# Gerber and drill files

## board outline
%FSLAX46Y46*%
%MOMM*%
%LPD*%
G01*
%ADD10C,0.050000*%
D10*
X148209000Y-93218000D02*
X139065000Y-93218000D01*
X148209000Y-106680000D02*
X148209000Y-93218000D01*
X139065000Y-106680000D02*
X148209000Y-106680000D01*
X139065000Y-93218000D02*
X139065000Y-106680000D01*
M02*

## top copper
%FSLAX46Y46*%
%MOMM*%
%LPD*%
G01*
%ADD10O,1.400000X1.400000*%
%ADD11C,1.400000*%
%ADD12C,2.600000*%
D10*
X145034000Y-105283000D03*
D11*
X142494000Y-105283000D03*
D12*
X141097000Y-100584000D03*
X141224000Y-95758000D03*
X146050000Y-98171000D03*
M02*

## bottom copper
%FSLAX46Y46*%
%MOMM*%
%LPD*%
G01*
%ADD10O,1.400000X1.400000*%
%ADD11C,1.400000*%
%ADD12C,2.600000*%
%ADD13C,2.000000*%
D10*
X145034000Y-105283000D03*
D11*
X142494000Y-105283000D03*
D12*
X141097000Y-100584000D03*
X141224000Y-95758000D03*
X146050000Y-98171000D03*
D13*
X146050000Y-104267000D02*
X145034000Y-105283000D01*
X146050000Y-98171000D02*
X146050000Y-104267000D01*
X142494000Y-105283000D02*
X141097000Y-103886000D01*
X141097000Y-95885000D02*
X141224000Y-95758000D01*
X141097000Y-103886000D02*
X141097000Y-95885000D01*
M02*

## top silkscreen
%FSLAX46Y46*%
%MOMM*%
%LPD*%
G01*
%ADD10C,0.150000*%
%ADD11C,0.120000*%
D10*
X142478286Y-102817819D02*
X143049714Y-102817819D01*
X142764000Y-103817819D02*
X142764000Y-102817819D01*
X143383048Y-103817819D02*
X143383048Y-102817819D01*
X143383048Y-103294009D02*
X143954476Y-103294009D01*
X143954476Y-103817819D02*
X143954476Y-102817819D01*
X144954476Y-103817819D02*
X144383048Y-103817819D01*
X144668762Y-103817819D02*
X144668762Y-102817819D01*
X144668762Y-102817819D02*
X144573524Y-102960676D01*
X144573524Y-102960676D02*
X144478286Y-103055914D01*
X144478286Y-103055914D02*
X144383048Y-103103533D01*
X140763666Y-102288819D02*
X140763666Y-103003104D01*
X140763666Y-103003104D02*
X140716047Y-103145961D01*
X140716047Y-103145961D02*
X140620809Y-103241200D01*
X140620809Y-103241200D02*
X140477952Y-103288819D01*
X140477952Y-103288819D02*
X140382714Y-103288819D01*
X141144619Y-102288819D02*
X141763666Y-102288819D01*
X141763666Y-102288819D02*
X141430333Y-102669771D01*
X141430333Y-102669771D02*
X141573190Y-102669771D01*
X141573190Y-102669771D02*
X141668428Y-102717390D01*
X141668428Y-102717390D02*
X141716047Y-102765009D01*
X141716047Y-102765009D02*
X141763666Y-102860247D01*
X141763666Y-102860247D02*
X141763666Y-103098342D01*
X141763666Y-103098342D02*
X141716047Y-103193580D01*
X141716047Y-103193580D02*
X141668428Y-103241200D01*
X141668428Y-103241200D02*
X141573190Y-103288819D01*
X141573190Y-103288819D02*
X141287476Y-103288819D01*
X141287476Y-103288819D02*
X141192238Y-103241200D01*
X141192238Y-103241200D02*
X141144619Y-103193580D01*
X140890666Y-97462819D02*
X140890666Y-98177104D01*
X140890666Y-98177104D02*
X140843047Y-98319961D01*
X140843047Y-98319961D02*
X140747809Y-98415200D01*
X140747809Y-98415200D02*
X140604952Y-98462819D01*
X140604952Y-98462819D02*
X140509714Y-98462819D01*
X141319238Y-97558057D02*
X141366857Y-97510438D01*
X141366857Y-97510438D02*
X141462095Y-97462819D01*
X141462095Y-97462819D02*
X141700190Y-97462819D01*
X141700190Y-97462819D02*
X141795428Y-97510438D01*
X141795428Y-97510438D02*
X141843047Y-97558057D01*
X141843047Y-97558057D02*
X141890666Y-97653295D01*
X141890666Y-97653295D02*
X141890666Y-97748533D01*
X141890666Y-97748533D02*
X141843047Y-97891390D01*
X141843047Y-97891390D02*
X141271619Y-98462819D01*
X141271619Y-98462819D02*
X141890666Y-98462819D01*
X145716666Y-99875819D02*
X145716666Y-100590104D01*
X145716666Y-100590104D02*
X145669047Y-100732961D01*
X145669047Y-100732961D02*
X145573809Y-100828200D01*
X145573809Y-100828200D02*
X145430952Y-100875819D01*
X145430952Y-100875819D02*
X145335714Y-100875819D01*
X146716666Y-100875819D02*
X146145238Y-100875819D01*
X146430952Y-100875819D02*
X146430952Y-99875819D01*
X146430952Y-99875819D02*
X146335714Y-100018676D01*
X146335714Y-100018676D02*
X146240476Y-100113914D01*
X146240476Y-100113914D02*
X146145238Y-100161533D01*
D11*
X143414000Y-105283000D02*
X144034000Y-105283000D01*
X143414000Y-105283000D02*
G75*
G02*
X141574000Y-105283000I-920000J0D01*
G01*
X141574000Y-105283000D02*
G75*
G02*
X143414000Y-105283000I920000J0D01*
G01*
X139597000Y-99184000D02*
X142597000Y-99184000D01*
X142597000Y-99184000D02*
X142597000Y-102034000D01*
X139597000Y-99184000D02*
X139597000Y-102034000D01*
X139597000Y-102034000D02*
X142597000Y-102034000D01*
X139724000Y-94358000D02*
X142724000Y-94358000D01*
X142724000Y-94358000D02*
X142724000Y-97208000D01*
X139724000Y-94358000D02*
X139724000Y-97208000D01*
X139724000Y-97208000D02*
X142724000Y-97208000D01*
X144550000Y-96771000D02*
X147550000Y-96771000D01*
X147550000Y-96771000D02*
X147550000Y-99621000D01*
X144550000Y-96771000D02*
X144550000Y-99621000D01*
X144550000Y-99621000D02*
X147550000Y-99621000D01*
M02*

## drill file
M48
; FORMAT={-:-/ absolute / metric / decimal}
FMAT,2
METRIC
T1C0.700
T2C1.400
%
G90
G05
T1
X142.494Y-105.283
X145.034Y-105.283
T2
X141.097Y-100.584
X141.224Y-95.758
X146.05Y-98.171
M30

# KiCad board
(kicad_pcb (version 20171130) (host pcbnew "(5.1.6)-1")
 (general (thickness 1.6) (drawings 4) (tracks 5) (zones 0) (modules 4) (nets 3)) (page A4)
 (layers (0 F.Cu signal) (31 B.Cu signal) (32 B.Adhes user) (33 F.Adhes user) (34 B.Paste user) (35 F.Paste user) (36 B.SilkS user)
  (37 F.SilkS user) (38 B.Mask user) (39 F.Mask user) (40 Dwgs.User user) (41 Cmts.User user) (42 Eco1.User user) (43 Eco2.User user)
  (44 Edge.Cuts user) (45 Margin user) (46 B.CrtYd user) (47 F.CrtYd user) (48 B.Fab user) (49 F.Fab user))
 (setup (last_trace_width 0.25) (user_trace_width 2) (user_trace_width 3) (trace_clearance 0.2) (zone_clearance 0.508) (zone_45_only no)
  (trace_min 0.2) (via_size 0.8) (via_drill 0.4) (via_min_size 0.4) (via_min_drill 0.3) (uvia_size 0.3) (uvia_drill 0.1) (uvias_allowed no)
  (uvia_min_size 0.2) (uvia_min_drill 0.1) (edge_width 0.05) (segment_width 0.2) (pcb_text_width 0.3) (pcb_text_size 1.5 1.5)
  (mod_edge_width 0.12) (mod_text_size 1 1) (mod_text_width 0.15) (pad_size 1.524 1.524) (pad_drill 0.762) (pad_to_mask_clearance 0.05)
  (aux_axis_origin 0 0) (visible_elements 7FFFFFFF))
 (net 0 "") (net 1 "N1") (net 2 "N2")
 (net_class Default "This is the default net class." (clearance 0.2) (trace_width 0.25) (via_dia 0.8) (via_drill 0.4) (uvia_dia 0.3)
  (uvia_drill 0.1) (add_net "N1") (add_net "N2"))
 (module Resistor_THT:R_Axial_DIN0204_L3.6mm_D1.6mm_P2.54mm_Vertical (layer F.Cu) (at 142.494 105.283)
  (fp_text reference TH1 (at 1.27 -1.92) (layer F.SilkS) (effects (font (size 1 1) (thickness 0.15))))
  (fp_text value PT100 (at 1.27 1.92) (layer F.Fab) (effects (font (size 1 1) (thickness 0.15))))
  (fp_line (start 0.92 0) (end 1.54 0) (layer F.SilkS) (width 0.12))
  (fp_circle (center 0 0) (end 0.92 0) (layer F.SilkS) (width 0.12))
  (pad 2 thru_hole oval (at 2.54 0) (size 1.4 1.4) (drill 0.7) (layers *.Cu *.Mask) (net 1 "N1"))
  (pad 1 thru_hole circle (at 0 0) (size 1.4 1.4) (drill 0.7) (layers *.Cu *.Mask) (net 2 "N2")))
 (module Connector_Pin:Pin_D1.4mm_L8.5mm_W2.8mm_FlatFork (layer F.Cu) (at 141.097 100.584)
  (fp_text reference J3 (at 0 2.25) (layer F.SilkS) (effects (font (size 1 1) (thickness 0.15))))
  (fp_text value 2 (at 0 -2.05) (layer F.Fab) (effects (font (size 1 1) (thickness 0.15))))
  (fp_line (start -1.5 -1.4) (end 1.5 -1.4) (layer F.SilkS) (width 0.12))
  (fp_line (start 1.5 -1.4) (end 1.5 1.45) (layer F.SilkS) (width 0.12))
  (fp_line (start -1.5 -1.4) (end -1.5 1.45) (layer F.SilkS) (width 0.12))
  (fp_line (start -1.5 1.45) (end 1.5 1.45) (layer F.SilkS) (width 0.12))
  (pad 1 thru_hole circle (at 0 0) (size 2.6 2.6) (drill 1.4) (layers *.Cu *.Mask) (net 2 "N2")))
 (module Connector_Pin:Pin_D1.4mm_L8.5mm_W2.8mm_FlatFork (layer F.Cu) (at 141.224 95.758)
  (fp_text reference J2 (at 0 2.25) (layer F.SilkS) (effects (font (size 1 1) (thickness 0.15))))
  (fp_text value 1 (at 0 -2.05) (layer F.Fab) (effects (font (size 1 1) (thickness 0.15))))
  (fp_line (start -1.5 -1.4) (end 1.5 -1.4) (layer F.SilkS) (width 0.12))
  (fp_line (start 1.5 -1.4) (end 1.5 1.45) (layer F.SilkS) (width 0.12))
  (fp_line (start -1.5 -1.4) (end -1.5 1.45) (layer F.SilkS) (width 0.12))
  (fp_line (start -1.5 1.45) (end 1.5 1.45) (layer F.SilkS) (width 0.12))
  (pad 1 thru_hole circle (at 0 0) (size 2.6 2.6) (drill 1.4) (layers *.Cu *.Mask) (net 2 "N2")))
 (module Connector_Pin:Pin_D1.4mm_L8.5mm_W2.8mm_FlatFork (layer F.Cu) (at 146.05 98.171)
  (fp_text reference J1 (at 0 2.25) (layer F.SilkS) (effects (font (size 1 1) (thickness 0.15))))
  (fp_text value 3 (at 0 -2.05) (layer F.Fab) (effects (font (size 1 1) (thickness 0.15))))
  (fp_line (start -1.5 -1.4) (end 1.5 -1.4) (layer F.SilkS) (width 0.12))
  (fp_line (start 1.5 -1.4) (end 1.5 1.45) (layer F.SilkS) (width 0.12))
  (fp_line (start -1.5 -1.4) (end -1.5 1.45) (layer F.SilkS) (width 0.12))
  (fp_line (start -1.5 1.45) (end 1.5 1.45) (layer F.SilkS) (width 0.12))
  (pad 1 thru_hole circle (at 0 0) (size 2.6 2.6) (drill 1.4) (layers *.Cu *.Mask) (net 1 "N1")))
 (gr_line (start 148.209 93.218) (end 139.065 93.218) (layer Edge.Cuts) (width 0.05))
 (gr_line (start 148.209 106.68) (end 148.209 93.218) (layer Edge.Cuts) (width 0.05))
 (gr_line (start 139.065 106.68) (end 148.209 106.68) (layer Edge.Cuts) (width 0.05))
 (gr_line (start 139.065 93.218) (end 139.065 106.68) (layer Edge.Cuts) (width 0.05))
 (segment (start 146.05 104.267) (end 145.034 105.283) (width 2) (layer B.Cu) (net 1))
 (segment (start 146.05 98.171) (end 146.05 104.267) (width 2) (layer B.Cu) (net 1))
 (segment (start 142.494 105.283) (end 141.097 103.886) (width 2) (layer B.Cu) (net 2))
 (segment (start 141.097 95.885) (end 141.224 95.758) (width 2) (layer B.Cu) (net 2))
 (segment (start 141.097 103.886) (end 141.097 95.885) (width 2) (layer B.Cu) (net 2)))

